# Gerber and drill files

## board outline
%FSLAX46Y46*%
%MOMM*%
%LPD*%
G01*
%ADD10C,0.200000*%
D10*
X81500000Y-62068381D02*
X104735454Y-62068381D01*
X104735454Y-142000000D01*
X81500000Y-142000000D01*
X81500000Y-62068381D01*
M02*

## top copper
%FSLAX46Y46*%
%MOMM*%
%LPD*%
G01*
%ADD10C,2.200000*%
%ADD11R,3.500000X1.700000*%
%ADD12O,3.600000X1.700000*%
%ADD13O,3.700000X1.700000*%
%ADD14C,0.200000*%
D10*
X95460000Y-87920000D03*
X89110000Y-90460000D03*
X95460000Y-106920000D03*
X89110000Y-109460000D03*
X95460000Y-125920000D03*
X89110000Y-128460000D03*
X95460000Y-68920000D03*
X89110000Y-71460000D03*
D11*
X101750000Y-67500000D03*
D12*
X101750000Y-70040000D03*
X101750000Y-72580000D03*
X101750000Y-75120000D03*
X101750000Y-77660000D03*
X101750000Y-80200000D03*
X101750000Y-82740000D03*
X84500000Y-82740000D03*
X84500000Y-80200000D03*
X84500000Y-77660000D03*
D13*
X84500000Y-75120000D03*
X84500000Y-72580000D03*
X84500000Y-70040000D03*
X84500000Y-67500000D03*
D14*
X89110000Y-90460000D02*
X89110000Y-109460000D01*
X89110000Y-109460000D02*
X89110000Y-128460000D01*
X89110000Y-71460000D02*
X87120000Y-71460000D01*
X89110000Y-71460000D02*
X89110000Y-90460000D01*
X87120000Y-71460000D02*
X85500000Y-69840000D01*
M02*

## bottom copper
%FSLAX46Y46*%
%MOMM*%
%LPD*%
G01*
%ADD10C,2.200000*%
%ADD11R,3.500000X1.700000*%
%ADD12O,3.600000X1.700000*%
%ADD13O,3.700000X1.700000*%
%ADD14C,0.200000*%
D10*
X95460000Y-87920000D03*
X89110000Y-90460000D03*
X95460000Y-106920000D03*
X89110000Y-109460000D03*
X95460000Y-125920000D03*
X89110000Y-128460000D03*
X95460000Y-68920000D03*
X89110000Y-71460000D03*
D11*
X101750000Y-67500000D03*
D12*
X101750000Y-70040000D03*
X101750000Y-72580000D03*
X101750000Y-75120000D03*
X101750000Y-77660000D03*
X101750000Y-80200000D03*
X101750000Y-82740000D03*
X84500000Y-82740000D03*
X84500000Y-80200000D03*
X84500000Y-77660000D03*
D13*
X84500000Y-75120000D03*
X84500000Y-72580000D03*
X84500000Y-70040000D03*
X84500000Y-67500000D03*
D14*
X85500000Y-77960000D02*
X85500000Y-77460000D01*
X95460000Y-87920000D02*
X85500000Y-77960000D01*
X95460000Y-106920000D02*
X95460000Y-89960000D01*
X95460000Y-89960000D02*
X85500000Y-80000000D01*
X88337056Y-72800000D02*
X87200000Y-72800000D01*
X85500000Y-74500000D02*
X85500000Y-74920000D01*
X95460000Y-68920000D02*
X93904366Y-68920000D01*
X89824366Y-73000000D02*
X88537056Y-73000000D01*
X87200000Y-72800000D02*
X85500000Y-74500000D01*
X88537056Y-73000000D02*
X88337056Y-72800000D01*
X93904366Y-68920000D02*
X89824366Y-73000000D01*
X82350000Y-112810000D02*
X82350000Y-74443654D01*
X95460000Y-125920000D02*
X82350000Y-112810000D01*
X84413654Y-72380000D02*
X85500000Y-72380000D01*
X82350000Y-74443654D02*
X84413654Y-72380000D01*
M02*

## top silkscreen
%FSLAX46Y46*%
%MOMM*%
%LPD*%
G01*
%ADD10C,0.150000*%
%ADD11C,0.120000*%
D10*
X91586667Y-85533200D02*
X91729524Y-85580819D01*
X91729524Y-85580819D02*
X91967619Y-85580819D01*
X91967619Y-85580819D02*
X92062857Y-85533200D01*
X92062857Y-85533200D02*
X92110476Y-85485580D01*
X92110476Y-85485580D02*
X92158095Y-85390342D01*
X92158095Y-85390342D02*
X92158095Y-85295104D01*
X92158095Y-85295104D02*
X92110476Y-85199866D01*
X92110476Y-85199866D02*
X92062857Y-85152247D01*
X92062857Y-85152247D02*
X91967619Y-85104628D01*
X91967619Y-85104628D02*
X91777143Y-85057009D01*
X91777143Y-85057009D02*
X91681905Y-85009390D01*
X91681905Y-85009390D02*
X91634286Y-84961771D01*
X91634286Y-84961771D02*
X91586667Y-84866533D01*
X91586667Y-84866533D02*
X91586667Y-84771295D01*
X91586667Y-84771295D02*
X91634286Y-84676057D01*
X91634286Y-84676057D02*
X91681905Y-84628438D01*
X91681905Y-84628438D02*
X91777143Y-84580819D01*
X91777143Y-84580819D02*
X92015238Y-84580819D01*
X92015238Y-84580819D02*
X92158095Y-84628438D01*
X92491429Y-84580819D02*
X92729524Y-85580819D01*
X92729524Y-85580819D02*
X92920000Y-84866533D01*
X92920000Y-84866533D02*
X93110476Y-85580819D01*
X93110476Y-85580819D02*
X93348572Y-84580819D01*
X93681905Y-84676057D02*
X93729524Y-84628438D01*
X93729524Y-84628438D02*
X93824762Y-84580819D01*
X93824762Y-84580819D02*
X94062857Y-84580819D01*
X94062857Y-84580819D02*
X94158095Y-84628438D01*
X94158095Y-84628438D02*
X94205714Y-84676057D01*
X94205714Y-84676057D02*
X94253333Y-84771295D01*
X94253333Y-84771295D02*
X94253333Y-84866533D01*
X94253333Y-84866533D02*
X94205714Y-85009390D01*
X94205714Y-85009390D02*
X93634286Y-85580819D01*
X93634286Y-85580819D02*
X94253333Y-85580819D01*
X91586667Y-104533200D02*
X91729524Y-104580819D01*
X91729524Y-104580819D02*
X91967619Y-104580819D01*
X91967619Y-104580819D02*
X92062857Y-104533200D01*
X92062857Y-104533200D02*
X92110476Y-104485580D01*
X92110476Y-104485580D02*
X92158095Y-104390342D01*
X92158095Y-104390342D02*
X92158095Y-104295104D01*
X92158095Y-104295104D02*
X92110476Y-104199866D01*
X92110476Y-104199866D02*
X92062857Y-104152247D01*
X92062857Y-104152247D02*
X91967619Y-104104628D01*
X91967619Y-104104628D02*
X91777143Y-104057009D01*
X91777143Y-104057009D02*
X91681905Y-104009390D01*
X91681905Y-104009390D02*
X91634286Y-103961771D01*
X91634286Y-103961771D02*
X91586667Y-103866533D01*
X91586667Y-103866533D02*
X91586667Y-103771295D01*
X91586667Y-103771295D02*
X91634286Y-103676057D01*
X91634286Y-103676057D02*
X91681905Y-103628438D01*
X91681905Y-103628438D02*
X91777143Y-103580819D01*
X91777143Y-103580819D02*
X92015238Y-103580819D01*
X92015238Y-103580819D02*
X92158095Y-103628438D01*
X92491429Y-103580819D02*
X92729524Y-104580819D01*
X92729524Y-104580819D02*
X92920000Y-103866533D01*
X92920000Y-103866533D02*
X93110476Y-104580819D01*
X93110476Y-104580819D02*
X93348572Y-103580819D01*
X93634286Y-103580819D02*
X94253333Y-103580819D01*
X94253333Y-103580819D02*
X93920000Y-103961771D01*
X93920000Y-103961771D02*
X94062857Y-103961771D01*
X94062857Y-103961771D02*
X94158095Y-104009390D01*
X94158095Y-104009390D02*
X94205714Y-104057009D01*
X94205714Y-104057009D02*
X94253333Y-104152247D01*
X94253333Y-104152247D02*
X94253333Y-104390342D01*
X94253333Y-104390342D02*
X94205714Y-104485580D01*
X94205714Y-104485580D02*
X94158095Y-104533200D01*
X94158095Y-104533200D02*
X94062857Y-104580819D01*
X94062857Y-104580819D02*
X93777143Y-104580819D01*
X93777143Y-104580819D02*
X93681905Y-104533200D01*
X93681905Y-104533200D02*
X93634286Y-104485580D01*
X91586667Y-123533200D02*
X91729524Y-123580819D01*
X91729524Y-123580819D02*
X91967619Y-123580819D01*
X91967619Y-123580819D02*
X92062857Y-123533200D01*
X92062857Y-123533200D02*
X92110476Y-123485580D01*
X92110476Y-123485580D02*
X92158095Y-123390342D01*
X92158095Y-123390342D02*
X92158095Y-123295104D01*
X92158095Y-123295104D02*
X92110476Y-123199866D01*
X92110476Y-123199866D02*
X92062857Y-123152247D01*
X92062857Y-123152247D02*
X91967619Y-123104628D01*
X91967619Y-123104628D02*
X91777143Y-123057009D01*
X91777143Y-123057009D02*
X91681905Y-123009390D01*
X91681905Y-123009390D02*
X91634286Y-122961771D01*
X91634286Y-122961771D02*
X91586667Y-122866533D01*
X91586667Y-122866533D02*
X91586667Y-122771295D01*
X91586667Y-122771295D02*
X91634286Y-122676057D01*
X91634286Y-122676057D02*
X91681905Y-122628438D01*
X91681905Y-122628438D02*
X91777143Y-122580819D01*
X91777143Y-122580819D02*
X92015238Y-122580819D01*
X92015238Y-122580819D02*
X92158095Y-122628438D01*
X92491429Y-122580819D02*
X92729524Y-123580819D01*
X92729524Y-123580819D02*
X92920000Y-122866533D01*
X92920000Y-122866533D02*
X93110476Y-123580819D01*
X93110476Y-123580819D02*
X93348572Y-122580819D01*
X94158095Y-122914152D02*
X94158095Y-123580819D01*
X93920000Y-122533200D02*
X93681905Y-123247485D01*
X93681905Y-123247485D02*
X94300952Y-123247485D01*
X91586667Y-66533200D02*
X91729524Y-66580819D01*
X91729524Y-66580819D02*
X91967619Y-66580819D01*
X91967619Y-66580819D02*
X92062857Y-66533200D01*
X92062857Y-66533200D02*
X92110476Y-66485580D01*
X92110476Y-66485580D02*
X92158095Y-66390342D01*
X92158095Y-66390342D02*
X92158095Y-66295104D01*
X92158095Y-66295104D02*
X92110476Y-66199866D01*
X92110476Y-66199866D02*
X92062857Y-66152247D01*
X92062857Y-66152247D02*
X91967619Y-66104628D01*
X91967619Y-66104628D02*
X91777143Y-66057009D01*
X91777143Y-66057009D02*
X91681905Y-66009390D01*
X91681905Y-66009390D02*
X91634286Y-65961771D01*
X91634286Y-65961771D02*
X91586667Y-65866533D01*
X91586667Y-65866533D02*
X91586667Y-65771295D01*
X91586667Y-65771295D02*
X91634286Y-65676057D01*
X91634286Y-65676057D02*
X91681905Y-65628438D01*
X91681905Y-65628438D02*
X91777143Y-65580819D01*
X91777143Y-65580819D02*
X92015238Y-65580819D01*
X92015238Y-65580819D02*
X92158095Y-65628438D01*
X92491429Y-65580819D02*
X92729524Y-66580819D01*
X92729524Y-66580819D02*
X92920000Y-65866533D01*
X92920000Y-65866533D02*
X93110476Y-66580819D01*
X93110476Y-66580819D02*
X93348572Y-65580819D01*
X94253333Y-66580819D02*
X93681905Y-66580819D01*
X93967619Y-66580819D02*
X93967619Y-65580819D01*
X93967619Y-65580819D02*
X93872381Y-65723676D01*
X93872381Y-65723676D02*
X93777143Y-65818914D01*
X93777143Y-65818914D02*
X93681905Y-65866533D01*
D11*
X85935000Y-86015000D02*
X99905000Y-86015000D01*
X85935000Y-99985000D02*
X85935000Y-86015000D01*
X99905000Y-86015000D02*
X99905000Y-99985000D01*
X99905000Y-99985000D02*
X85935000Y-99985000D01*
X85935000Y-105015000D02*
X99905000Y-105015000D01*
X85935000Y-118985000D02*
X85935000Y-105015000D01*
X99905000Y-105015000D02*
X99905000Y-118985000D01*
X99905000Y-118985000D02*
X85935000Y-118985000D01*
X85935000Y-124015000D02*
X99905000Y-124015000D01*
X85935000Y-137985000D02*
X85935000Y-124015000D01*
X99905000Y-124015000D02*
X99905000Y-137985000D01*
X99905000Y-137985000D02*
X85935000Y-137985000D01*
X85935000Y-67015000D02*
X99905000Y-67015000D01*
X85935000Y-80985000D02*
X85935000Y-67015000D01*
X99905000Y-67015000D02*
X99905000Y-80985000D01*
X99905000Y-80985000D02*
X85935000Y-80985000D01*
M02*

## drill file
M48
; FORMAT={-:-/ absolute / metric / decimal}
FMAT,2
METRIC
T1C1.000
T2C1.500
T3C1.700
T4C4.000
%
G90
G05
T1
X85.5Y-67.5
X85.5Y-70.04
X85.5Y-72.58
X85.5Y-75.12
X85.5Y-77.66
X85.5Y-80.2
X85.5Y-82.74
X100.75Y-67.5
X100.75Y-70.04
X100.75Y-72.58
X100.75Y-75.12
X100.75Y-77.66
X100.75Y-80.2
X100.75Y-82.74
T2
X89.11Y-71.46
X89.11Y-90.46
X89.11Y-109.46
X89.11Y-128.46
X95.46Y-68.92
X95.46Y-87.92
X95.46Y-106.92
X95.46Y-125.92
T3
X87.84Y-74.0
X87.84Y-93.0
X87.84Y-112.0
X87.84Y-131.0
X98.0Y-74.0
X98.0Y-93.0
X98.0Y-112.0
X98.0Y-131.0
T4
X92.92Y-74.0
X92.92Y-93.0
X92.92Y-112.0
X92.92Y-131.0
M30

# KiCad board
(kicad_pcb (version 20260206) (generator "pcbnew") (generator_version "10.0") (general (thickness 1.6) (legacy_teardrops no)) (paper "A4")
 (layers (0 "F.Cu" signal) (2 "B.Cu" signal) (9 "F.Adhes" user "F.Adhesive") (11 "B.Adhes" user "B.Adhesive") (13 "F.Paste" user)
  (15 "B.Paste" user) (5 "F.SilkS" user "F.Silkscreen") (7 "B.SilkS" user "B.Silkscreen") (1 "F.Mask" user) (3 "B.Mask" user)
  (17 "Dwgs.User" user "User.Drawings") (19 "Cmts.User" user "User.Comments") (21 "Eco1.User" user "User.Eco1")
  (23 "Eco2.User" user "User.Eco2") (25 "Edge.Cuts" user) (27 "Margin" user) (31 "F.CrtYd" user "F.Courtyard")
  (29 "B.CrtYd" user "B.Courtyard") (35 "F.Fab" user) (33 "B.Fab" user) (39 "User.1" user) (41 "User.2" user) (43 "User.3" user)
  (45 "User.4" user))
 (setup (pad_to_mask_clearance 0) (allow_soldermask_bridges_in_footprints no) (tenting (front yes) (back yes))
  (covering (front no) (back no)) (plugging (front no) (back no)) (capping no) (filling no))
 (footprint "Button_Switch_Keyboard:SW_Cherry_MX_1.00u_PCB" (layer "F.Cu") (at 95.46 87.92)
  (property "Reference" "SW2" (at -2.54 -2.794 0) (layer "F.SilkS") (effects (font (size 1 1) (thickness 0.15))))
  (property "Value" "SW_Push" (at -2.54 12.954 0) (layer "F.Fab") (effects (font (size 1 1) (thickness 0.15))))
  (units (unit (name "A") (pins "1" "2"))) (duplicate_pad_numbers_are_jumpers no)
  (fp_line (start -9.525 -1.905) (end 4.445 -1.905) (stroke (width 0.12) (type solid)) (layer "F.SilkS"))
  (fp_line (start -9.525 12.065) (end -9.525 -1.905) (stroke (width 0.12) (type solid)) (layer "F.SilkS"))
  (fp_line (start 4.445 -1.905) (end 4.445 12.065) (stroke (width 0.12) (type solid)) (layer "F.SilkS"))
  (fp_line (start 4.445 12.065) (end -9.525 12.065) (stroke (width 0.12) (type solid)) (layer "F.SilkS"))
  (pad "" np_thru_hole circle (at -7.62 5.08) (size 1.7 1.7) (drill 1.7) (layers "*.Cu" "*.Mask"))
  (pad "" np_thru_hole circle (at -2.54 5.08) (size 4 4) (drill 4) (layers "*.Cu" "*.Mask"))
  (pad "" np_thru_hole circle (at 2.54 5.08) (size 1.7 1.7) (drill 1.7) (layers "*.Cu" "*.Mask"))
  (pad "1" thru_hole circle (at 0 0) (size 2.2 2.2) (drill 1.5) (layers "*.Cu" "*.Mask") (remove_unused_layers no)
   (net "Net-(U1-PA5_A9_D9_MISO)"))
  (pad "2" thru_hole circle (at -6.35 2.54) (size 2.2 2.2) (drill 1.5) (layers "*.Cu" "*.Mask") (remove_unused_layers no) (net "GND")))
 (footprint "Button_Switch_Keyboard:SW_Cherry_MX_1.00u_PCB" (layer "F.Cu") (at 95.46 106.92)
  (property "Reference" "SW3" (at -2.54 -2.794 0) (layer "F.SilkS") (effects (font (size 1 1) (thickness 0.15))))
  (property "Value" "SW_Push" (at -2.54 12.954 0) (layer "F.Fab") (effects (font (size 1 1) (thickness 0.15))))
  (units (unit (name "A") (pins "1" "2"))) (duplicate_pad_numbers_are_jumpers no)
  (fp_line (start -9.525 -1.905) (end 4.445 -1.905) (stroke (width 0.12) (type solid)) (layer "F.SilkS"))
  (fp_line (start -9.525 12.065) (end -9.525 -1.905) (stroke (width 0.12) (type solid)) (layer "F.SilkS"))
  (fp_line (start 4.445 -1.905) (end 4.445 12.065) (stroke (width 0.12) (type solid)) (layer "F.SilkS"))
  (fp_line (start 4.445 12.065) (end -9.525 12.065) (stroke (width 0.12) (type solid)) (layer "F.SilkS"))
  (pad "" np_thru_hole circle (at -7.62 5.08) (size 1.7 1.7) (drill 1.7) (layers "*.Cu" "*.Mask"))
  (pad "" np_thru_hole circle (at -2.54 5.08) (size 4 4) (drill 4) (layers "*.Cu" "*.Mask"))
  (pad "" np_thru_hole circle (at 2.54 5.08) (size 1.7 1.7) (drill 1.7) (layers "*.Cu" "*.Mask"))
  (pad "1" thru_hole circle (at 0 0) (size 2.2 2.2) (drill 1.5) (layers "*.Cu" "*.Mask") (remove_unused_layers no)
   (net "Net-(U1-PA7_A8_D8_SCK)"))
  (pad "2" thru_hole circle (at -6.35 2.54) (size 2.2 2.2) (drill 1.5) (layers "*.Cu" "*.Mask") (remove_unused_layers no) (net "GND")))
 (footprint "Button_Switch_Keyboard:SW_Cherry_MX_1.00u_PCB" (layer "F.Cu") (at 95.46 125.92)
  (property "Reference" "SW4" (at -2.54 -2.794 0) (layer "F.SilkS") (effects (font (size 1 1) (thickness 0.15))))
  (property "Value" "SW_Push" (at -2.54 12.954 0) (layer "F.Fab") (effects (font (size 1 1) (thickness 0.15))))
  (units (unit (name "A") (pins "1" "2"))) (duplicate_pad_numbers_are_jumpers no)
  (fp_line (start -9.525 -1.905) (end 4.445 -1.905) (stroke (width 0.12) (type solid)) (layer "F.SilkS"))
  (fp_line (start -9.525 12.065) (end -9.525 -1.905) (stroke (width 0.12) (type solid)) (layer "F.SilkS"))
  (fp_line (start 4.445 -1.905) (end 4.445 12.065) (stroke (width 0.12) (type solid)) (layer "F.SilkS"))
  (fp_line (start 4.445 12.065) (end -9.525 12.065) (stroke (width 0.12) (type solid)) (layer "F.SilkS"))
  (pad "" np_thru_hole circle (at -7.62 5.08) (size 1.7 1.7) (drill 1.7) (layers "*.Cu" "*.Mask"))
  (pad "" np_thru_hole circle (at -2.54 5.08) (size 4 4) (drill 4) (layers "*.Cu" "*.Mask"))
  (pad "" np_thru_hole circle (at 2.54 5.08) (size 1.7 1.7) (drill 1.7) (layers "*.Cu" "*.Mask"))
  (pad "1" thru_hole circle (at 0 0) (size 2.2 2.2) (drill 1.5) (layers "*.Cu" "*.Mask") (remove_unused_layers no) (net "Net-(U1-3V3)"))
  (pad "2" thru_hole circle (at -6.35 2.54) (size 2.2 2.2) (drill 1.5) (layers "*.Cu" "*.Mask") (remove_unused_layers no) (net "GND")))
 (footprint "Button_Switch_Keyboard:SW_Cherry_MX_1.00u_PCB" (layer "F.Cu") (at 95.46 68.92)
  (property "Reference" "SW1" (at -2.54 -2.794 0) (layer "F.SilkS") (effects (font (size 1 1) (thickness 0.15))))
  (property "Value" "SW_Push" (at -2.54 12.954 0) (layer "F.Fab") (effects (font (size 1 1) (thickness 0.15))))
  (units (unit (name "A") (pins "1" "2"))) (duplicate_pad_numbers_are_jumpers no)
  (fp_line (start -9.525 -1.905) (end 4.445 -1.905) (stroke (width 0.12) (type solid)) (layer "F.SilkS"))
  (fp_line (start -9.525 12.065) (end -9.525 -1.905) (stroke (width 0.12) (type solid)) (layer "F.SilkS"))
  (fp_line (start 4.445 -1.905) (end 4.445 12.065) (stroke (width 0.12) (type solid)) (layer "F.SilkS"))
  (fp_line (start 4.445 12.065) (end -9.525 12.065) (stroke (width 0.12) (type solid)) (layer "F.SilkS"))
  (pad "" np_thru_hole circle (at -7.62 5.08) (size 1.7 1.7) (drill 1.7) (layers "*.Cu" "*.Mask"))
  (pad "" np_thru_hole circle (at -2.54 5.08) (size 4 4) (drill 4) (layers "*.Cu" "*.Mask"))
  (pad "" np_thru_hole circle (at 2.54 5.08) (size 1.7 1.7) (drill 1.7) (layers "*.Cu" "*.Mask"))
  (pad "1" thru_hole circle (at 0 0) (size 2.2 2.2) (drill 1.5) (layers "*.Cu" "*.Mask") (remove_unused_layers no)
   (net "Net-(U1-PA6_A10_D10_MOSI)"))
  (pad "2" thru_hole circle (at -6.35 2.54) (size 2.2 2.2) (drill 1.5) (layers "*.Cu" "*.Mask") (remove_unused_layers no) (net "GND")))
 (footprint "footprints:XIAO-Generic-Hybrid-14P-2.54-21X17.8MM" (layer "B.Cu") (at 93.125 75.12 180)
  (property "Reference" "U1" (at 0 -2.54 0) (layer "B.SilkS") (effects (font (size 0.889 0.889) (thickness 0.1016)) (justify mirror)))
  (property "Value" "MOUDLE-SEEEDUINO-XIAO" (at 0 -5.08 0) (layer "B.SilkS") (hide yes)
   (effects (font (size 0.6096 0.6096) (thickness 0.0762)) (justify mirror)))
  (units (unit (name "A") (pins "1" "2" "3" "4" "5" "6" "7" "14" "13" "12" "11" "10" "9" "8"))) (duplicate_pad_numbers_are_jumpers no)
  (pad "1" thru_hole rect (at -7.625 7.62 180) (size 3.5 1.7) (drill 1 (offset -1 0)) (layers "*.Cu" "*.Mask") (remove_unused_layers no)
   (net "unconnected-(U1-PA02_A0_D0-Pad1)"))
  (pad "2" thru_hole oval (at -7.625 5.08 180) (size 3.6 1.7) (drill 1 (offset -1 0)) (layers "*.Cu" "*.Mask") (remove_unused_layers no)
   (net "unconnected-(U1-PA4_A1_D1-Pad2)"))
  (pad "3" thru_hole oval (at -7.625 2.54 180) (size 3.6 1.7) (drill 1 (offset -1 0)) (layers "*.Cu" "*.Mask") (remove_unused_layers no)
   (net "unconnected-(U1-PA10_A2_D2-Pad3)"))
  (pad "4" thru_hole oval (at -7.625 0 180) (size 3.6 1.7) (drill 1 (offset -1 0)) (layers "*.Cu" "*.Mask") (remove_unused_layers no)
   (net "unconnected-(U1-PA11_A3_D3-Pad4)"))
  (pad "5" thru_hole oval (at -7.625 -2.54 180) (size 3.6 1.7) (drill 1 (offset -1 0)) (layers "*.Cu" "*.Mask") (remove_unused_layers no)
   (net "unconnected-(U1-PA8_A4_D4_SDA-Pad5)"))
  (pad "6" thru_hole oval (at -7.625 -5.08) (size 3.6 1.7) (drill 1 (offset 1 0)) (layers "*.Cu" "*.Mask") (remove_unused_layers no)
   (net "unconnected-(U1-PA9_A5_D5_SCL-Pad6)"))
  (pad "7" thru_hole oval (at -7.625 -7.62 180) (size 3.6 1.7) (drill 1 (offset -1 0)) (layers "*.Cu" "*.Mask") (remove_unused_layers no)
   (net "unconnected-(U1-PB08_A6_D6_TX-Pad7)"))
  (pad "8" thru_hole oval (at 7.625 -7.62 180) (size 3.6 1.7) (drill 1 (offset 1 0)) (layers "*.Cu" "*.Mask") (remove_unused_layers no)
   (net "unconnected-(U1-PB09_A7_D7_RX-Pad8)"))
  (pad "9" thru_hole oval (at 7.625 -5.08 180) (size 3.6 1.7) (drill 1 (offset 1 0)) (layers "*.Cu" "*.Mask") (remove_unused_layers no)
   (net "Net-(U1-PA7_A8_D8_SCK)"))
  (pad "10" thru_hole oval (at 7.625 -2.54 180) (size 3.6 1.7) (drill 1 (offset 1 0)) (layers "*.Cu" "*.Mask") (remove_unused_layers no)
   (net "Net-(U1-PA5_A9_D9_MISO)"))
  (pad "11" thru_hole oval (at 7.625 0 180) (size 3.7 1.7) (drill 1 (offset 1 0)) (layers "*.Cu" "*.Mask") (remove_unused_layers no)
   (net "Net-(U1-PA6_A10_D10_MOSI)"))
  (pad "12" thru_hole oval (at 7.625 2.54 180) (size 3.7 1.7) (drill 1 (offset 1 0)) (layers "*.Cu" "*.Mask") (remove_unused_layers no)
   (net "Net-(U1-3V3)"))
  (pad "13" thru_hole oval (at 7.625 5.08 180) (size 3.7 1.7) (drill 1 (offset 1 0)) (layers "*.Cu" "*.Mask") (remove_unused_layers no)
   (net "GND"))
  (pad "14" thru_hole oval (at 7.625 7.62 180) (size 3.7 1.7) (drill 1 (offset 1 0)) (layers "*.Cu" "*.Mask") (remove_unused_layers no)
   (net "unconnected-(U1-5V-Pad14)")))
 (gr_rect (start 81.5 62.068381) (end 104.735454 142) (stroke (width 0.2) (type solid)) (fill no) (layer "Edge.Cuts"))
 (segment (start 85.5 77.96) (end 85.5 77.46) (width 0.2) (layer "B.Cu") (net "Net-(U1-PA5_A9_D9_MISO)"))
 (segment (start 95.46 87.92) (end 85.5 77.96) (width 0.2) (layer "B.Cu") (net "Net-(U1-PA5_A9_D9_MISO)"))
 (segment (start 89.11 90.46) (end 89.11 109.46) (width 0.2) (layer "F.Cu") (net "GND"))
 (segment (start 89.11 109.46) (end 89.11 128.46) (width 0.2) (layer "F.Cu") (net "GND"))
 (segment (start 89.11 71.46) (end 87.12 71.46) (width 0.2) (layer "F.Cu") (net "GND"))
 (segment (start 89.11 71.46) (end 89.11 90.46) (width 0.2) (layer "F.Cu") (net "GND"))
 (segment (start 87.12 71.46) (end 85.5 69.84) (width 0.2) (layer "F.Cu") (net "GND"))
 (segment (start 95.46 106.92) (end 95.46 89.96) (width 0.2) (layer "B.Cu") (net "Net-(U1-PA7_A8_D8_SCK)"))
 (segment (start 95.46 89.96) (end 85.5 80) (width 0.2) (layer "B.Cu") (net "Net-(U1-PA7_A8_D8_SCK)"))
 (segment (start 88.337056 72.8) (end 87.2 72.8) (width 0.2) (layer "B.Cu") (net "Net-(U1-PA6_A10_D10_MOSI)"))
 (segment (start 85.5 74.5) (end 85.5 74.92) (width 0.2) (layer "B.Cu") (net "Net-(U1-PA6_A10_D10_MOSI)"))
 (segment (start 95.46 68.92) (end 93.904366 68.92) (width 0.2) (layer "B.Cu") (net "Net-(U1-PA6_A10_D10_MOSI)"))
 (segment (start 89.824366 73) (end 88.537056 73) (width 0.2) (layer "B.Cu") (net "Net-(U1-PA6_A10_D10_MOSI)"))
 (segment (start 87.2 72.8) (end 85.5 74.5) (width 0.2) (layer "B.Cu") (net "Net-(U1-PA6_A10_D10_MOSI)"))
 (segment (start 88.537056 73) (end 88.337056 72.8) (width 0.2) (layer "B.Cu") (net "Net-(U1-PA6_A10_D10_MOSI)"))
 (segment (start 93.904366 68.92) (end 89.824366 73) (width 0.2) (layer "B.Cu") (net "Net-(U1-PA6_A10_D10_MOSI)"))
 (segment (start 82.35 112.81) (end 82.35 74.443654) (width 0.2) (layer "B.Cu") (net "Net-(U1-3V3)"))
 (segment (start 95.46 125.92) (end 82.35 112.81) (width 0.2) (layer "B.Cu") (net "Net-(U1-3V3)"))
 (segment (start 84.413654 72.38) (end 85.5 72.38) (width 0.2) (layer "B.Cu") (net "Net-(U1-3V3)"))
 (segment (start 82.35 74.443654) (end 84.413654 72.38) (width 0.2) (layer "B.Cu") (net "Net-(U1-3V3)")))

